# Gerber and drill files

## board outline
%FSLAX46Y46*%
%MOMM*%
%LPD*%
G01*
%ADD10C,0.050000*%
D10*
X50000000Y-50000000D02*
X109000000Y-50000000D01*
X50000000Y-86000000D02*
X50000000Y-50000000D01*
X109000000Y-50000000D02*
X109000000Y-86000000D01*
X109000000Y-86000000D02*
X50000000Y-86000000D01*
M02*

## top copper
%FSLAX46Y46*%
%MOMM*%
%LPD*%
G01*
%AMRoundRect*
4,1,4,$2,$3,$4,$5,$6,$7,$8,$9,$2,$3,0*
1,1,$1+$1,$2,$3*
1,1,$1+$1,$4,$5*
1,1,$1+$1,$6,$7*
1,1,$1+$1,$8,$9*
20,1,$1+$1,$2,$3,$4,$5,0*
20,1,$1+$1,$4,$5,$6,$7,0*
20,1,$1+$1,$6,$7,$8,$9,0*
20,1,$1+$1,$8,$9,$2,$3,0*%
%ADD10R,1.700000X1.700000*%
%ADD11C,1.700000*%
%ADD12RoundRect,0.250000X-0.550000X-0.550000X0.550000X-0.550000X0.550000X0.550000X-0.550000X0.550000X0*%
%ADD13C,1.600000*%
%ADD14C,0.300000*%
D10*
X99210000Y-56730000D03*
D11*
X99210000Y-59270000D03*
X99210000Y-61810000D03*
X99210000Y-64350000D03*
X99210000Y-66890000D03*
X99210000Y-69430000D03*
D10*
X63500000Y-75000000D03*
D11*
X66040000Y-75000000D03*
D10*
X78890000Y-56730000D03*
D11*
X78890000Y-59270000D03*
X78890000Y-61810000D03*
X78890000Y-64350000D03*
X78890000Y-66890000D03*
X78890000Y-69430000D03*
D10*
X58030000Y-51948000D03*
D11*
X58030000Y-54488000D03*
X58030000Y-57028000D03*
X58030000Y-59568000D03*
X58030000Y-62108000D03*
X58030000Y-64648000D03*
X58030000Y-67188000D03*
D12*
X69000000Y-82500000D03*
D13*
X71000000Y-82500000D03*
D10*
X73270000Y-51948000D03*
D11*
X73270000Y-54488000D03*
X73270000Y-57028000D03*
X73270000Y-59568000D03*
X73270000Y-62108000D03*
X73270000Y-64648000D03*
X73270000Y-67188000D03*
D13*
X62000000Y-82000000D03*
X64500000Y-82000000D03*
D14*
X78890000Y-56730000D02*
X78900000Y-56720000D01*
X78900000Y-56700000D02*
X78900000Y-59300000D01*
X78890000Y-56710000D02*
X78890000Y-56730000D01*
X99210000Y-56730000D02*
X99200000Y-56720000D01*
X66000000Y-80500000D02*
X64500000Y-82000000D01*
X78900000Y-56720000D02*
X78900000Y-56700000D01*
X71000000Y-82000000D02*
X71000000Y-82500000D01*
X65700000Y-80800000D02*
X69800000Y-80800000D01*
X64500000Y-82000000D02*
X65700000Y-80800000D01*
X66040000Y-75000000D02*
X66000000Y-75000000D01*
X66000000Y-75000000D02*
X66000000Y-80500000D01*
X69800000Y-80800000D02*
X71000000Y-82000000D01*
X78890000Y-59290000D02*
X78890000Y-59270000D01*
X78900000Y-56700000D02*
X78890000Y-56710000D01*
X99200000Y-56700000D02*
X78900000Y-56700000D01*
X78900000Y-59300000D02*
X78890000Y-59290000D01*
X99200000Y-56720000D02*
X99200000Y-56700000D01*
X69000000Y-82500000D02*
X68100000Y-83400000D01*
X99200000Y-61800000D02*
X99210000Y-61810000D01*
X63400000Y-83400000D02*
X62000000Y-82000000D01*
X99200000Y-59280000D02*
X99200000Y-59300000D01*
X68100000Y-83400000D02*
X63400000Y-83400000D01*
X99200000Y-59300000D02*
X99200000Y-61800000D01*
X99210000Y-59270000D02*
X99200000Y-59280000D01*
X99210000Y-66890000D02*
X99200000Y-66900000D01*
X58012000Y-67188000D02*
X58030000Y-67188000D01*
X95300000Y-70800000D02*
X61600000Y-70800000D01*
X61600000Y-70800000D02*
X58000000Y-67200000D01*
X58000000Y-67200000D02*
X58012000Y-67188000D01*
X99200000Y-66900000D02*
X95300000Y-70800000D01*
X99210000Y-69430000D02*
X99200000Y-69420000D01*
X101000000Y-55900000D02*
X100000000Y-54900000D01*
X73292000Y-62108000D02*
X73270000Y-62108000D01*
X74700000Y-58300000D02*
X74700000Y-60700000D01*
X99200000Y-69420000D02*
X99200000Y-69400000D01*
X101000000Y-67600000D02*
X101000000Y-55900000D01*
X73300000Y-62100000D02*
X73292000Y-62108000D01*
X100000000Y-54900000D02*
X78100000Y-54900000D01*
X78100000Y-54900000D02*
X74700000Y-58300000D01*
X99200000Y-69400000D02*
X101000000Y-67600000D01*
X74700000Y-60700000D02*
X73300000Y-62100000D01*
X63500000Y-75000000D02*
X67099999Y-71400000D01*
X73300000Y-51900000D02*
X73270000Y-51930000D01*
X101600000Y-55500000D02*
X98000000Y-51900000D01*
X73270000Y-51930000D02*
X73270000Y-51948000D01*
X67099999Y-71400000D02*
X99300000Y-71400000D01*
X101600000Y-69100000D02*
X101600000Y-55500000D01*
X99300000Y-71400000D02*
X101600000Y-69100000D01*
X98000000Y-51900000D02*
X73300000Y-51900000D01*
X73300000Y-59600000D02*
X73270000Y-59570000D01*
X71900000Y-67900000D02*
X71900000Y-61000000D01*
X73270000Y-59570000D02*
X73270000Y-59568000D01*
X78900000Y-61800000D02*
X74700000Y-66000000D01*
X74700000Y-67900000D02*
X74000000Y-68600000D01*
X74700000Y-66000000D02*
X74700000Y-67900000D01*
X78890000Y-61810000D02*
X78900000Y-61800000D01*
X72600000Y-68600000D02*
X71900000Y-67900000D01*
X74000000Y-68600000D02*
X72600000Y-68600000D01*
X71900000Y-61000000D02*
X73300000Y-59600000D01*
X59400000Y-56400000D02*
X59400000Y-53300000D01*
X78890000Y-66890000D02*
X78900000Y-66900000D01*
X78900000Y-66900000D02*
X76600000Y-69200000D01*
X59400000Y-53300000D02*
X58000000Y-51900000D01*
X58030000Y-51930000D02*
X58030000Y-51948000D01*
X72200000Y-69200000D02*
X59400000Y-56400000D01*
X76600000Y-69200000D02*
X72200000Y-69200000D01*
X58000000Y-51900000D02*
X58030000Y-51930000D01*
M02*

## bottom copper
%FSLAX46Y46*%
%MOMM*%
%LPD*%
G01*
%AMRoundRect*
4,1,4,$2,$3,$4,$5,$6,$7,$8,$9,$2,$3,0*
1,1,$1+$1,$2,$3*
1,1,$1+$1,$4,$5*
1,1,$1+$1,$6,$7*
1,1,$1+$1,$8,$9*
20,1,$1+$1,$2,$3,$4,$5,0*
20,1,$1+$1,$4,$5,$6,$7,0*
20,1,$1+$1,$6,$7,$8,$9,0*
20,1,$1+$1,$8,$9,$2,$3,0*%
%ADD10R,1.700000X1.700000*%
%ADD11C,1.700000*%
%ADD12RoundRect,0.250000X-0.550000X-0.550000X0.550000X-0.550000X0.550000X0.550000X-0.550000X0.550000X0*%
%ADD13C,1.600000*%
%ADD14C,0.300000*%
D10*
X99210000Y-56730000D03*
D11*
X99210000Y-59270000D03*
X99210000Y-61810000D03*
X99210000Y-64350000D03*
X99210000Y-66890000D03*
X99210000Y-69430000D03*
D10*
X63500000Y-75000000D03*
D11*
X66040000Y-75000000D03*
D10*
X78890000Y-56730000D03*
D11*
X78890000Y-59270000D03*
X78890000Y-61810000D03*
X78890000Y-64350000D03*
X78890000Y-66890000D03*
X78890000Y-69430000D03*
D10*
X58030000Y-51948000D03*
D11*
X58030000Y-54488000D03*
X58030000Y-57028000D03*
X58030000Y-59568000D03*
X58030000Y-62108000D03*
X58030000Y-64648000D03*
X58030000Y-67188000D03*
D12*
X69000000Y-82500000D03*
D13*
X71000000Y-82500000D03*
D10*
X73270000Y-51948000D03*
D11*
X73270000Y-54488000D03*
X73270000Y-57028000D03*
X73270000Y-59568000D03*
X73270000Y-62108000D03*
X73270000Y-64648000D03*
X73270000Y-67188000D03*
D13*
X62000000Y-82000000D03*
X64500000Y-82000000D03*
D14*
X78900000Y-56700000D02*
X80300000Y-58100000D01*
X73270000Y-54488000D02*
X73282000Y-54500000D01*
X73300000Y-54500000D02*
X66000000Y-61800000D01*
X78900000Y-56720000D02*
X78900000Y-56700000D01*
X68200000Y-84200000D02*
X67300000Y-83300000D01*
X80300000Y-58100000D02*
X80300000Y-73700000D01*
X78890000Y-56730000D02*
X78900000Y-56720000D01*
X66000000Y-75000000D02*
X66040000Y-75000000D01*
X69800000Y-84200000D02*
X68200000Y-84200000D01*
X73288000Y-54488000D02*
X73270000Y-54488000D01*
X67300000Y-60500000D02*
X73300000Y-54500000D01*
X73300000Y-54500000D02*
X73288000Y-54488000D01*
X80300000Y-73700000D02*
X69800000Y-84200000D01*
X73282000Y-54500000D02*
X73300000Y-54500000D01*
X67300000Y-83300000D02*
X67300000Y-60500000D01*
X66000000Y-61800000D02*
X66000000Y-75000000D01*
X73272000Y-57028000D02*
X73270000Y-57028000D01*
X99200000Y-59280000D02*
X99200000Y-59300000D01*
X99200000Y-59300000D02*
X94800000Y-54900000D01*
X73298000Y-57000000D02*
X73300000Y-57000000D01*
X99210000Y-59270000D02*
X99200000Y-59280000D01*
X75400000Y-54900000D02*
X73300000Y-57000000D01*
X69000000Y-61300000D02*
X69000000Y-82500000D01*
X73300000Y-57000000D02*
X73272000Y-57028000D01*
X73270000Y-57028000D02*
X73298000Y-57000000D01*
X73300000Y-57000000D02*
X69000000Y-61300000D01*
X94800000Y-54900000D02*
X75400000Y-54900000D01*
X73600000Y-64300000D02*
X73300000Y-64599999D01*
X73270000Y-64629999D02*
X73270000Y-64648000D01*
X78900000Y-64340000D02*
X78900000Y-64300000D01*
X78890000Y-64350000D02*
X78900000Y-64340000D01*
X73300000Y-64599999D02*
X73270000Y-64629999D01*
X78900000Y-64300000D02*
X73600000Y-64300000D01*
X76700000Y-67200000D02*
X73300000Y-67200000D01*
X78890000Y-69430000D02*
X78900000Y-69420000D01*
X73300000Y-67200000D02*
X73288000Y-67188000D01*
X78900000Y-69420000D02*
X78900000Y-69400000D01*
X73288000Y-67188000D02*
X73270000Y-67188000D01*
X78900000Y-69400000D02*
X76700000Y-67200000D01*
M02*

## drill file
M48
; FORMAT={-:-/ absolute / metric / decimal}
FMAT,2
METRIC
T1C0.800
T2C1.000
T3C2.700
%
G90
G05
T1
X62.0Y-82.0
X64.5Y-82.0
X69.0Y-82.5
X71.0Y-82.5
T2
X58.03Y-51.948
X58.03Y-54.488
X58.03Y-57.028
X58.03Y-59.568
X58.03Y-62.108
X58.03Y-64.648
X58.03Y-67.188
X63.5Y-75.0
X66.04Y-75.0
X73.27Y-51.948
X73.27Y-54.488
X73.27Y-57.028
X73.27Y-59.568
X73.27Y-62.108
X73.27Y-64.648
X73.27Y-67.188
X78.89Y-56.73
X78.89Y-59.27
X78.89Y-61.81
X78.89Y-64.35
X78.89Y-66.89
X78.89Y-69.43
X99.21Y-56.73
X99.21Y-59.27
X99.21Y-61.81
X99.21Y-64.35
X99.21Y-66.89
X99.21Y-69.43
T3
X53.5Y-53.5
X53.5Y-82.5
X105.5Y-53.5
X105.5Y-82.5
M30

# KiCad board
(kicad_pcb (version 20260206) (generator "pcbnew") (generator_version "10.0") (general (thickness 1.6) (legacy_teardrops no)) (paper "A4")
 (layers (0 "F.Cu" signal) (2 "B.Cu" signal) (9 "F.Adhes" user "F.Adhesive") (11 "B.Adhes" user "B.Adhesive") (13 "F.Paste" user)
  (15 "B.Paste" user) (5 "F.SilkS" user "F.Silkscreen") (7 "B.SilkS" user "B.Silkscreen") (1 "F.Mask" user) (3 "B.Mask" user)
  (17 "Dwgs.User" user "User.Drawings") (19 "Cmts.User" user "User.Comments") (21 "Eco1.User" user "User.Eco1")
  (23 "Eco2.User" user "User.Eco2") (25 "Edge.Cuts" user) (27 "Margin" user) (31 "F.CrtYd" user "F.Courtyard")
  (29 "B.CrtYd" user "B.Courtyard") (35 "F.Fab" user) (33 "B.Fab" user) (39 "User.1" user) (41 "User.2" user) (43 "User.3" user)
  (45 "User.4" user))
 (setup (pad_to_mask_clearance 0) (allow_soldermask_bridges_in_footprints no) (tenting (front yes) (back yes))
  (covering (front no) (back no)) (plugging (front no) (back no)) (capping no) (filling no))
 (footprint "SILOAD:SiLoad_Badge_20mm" (layer "F.Cu") (at 89.05 82)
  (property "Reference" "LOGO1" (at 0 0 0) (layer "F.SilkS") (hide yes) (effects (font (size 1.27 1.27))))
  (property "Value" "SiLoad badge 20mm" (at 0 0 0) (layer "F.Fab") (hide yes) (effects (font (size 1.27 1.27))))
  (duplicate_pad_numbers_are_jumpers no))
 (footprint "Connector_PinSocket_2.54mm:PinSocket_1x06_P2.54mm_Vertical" (layer "F.Cu") (at 99.21 56.73)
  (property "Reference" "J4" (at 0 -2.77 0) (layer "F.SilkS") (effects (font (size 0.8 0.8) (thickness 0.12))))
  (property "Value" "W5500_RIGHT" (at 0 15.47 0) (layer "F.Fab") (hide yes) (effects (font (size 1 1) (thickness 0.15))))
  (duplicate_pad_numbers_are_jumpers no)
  (pad "1" thru_hole rect (at 0 0) (size 1.7 1.7) (drill 1) (layers "*.Cu" "*.Mask") (remove_unused_layers no) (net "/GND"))
  (pad "2" thru_hole circle (at 0 2.54) (size 1.7 1.7) (drill 1) (layers "*.Cu" "*.Mask") (remove_unused_layers no) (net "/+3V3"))
  (pad "3" thru_hole circle (at 0 5.08) (size 1.7 1.7) (drill 1) (layers "*.Cu" "*.Mask") (remove_unused_layers no) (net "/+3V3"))
  (pad "4" thru_hole circle (at 0 7.62) (size 1.7 1.7) (drill 1) (layers "*.Cu" "*.Mask") (remove_unused_layers no))
  (pad "5" thru_hole circle (at 0 10.16) (size 1.7 1.7) (drill 1) (layers "*.Cu" "*.Mask") (remove_unused_layers no) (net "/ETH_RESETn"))
  (pad "6" thru_hole circle (at 0 12.7) (size 1.7 1.7) (drill 1) (layers "*.Cu" "*.Mask") (remove_unused_layers no) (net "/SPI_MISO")))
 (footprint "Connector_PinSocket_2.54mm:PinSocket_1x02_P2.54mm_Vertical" (layer "F.Cu") (at 63.5 75 90)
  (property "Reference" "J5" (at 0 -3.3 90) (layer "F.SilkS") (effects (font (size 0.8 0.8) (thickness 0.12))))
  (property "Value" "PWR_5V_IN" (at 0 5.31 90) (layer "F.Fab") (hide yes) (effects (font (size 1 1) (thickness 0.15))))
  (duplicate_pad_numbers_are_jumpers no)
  (pad "1" thru_hole rect (at 0 0 90) (size 1.7 1.7) (drill 1) (layers "*.Cu" "*.Mask") (remove_unused_layers no) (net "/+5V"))
  (pad "2" thru_hole circle (at 0 2.54 90) (size 1.7 1.7) (drill 1) (layers "*.Cu" "*.Mask") (remove_unused_layers no) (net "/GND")))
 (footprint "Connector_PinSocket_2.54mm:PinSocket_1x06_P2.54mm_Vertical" (layer "F.Cu") (at 78.89 56.73)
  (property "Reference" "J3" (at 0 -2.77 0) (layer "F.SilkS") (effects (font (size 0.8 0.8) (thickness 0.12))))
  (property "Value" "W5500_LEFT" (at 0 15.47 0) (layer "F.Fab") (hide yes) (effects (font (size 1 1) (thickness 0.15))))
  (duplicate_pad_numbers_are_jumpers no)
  (pad "1" thru_hole rect (at 0 0) (size 1.7 1.7) (drill 1) (layers "*.Cu" "*.Mask") (remove_unused_layers no) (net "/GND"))
  (pad "2" thru_hole circle (at 0 2.54) (size 1.7 1.7) (drill 1) (layers "*.Cu" "*.Mask") (remove_unused_layers no) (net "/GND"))
  (pad "3" thru_hole circle (at 0 5.08) (size 1.7 1.7) (drill 1) (layers "*.Cu" "*.Mask") (remove_unused_layers no) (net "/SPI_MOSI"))
  (pad "4" thru_hole circle (at 0 7.62) (size 1.7 1.7) (drill 1) (layers "*.Cu" "*.Mask") (remove_unused_layers no) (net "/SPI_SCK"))
  (pad "5" thru_hole circle (at 0 10.16) (size 1.7 1.7) (drill 1) (layers "*.Cu" "*.Mask") (remove_unused_layers no) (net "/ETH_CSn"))
  (pad "6" thru_hole circle (at 0 12.7) (size 1.7 1.7) (drill 1) (layers "*.Cu" "*.Mask") (remove_unused_layers no) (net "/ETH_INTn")))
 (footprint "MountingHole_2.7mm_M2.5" (layer "F.Cu") (at 105.5 53.5)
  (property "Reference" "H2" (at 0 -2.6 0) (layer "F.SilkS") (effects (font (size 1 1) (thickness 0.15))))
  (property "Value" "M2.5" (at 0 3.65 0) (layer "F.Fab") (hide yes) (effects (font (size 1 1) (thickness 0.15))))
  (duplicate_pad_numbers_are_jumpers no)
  (pad "" np_thru_hole circle (at 0 0) (size 2.7 2.7) (drill 2.7) (layers "*.Cu" "*.Mask")))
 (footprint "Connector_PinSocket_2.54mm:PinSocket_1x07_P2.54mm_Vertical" (layer "F.Cu") (at 58.03 51.948)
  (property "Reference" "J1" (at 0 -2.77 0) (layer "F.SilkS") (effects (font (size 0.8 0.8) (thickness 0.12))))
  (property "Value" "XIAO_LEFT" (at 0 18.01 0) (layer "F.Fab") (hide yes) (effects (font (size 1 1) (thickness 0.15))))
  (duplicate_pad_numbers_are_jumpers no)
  (pad "1" thru_hole rect (at 0 0) (size 1.7 1.7) (drill 1) (layers "*.Cu" "*.Mask") (remove_unused_layers no) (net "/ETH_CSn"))
  (pad "2" thru_hole circle (at 0 2.54) (size 1.7 1.7) (drill 1) (layers "*.Cu" "*.Mask") (remove_unused_layers no))
  (pad "3" thru_hole circle (at 0 5.08) (size 1.7 1.7) (drill 1) (layers "*.Cu" "*.Mask") (remove_unused_layers no))
  (pad "4" thru_hole circle (at 0 7.62) (size 1.7 1.7) (drill 1) (layers "*.Cu" "*.Mask") (remove_unused_layers no))
  (pad "5" thru_hole circle (at 0 10.16) (size 1.7 1.7) (drill 1) (layers "*.Cu" "*.Mask") (remove_unused_layers no))
  (pad "6" thru_hole circle (at 0 12.7) (size 1.7 1.7) (drill 1) (layers "*.Cu" "*.Mask") (remove_unused_layers no))
  (pad "7" thru_hole circle (at 0 15.24) (size 1.7 1.7) (drill 1) (layers "*.Cu" "*.Mask") (remove_unused_layers no) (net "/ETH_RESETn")))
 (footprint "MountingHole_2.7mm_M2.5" (layer "F.Cu") (at 105.5 82.5)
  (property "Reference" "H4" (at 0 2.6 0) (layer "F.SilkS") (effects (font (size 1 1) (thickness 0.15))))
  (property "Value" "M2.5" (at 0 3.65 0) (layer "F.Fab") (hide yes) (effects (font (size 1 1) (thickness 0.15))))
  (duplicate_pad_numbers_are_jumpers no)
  (pad "" np_thru_hole circle (at 0 0) (size 2.7 2.7) (drill 2.7) (layers "*.Cu" "*.Mask")))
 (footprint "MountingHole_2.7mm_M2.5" (layer "F.Cu") (at 53.5 53.5)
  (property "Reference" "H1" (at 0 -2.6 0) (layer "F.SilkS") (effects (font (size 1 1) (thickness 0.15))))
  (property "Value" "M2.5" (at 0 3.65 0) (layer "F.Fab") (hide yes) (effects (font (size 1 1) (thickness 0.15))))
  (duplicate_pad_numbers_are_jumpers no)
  (pad "" np_thru_hole circle (at 0 0) (size 2.7 2.7) (drill 2.7) (layers "*.Cu" "*.Mask")))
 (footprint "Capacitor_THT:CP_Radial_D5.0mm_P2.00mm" (layer "F.Cu") (at 69 82.5)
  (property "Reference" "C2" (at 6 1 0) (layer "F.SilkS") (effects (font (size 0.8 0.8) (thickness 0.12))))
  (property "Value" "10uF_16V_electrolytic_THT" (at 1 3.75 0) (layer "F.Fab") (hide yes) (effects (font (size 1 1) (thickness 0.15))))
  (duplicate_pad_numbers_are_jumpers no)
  (pad "1" thru_hole roundrect (at 0 0) (size 1.6 1.6) (drill 0.8) (layers "*.Cu" "*.Mask") (remove_unused_layers no)
   (roundrect_rratio 0.15625) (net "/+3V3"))
  (pad "2" thru_hole circle (at 2 0) (size 1.6 1.6) (drill 0.8) (layers "*.Cu" "*.Mask") (remove_unused_layers no) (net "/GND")))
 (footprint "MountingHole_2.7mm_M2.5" (layer "F.Cu") (at 53.5 82.5)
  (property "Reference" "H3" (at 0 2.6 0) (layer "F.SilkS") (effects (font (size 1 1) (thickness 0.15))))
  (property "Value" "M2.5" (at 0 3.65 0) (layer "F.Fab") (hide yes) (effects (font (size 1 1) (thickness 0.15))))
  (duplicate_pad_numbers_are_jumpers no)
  (pad "" np_thru_hole circle (at 0 0) (size 2.7 2.7) (drill 2.7) (layers "*.Cu" "*.Mask")))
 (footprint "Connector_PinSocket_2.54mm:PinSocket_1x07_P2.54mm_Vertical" (layer "F.Cu") (at 73.27 51.948)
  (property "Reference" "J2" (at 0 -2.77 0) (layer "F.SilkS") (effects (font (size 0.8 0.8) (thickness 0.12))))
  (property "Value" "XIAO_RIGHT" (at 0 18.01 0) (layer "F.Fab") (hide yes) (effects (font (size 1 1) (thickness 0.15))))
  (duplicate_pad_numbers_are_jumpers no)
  (pad "1" thru_hole rect (at 0 0) (size 1.7 1.7) (drill 1) (layers "*.Cu" "*.Mask") (remove_unused_layers no) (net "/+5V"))
  (pad "2" thru_hole circle (at 0 2.54) (size 1.7 1.7) (drill 1) (layers "*.Cu" "*.Mask") (remove_unused_layers no) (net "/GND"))
  (pad "3" thru_hole circle (at 0 5.08) (size 1.7 1.7) (drill 1) (layers "*.Cu" "*.Mask") (remove_unused_layers no) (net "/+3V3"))
  (pad "4" thru_hole circle (at 0 7.62) (size 1.7 1.7) (drill 1) (layers "*.Cu" "*.Mask") (remove_unused_layers no) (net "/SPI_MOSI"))
  (pad "5" thru_hole circle (at 0 10.16) (size 1.7 1.7) (drill 1) (layers "*.Cu" "*.Mask") (remove_unused_layers no) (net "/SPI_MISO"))
  (pad "6" thru_hole circle (at 0 12.7) (size 1.7 1.7) (drill 1) (layers "*.Cu" "*.Mask") (remove_unused_layers no) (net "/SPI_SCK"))
  (pad "7" thru_hole circle (at 0 15.24) (size 1.7 1.7) (drill 1) (layers "*.Cu" "*.Mask") (remove_unused_layers no) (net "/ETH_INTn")))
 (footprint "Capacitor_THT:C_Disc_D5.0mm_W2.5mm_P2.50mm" (layer "F.Cu") (at 62 82)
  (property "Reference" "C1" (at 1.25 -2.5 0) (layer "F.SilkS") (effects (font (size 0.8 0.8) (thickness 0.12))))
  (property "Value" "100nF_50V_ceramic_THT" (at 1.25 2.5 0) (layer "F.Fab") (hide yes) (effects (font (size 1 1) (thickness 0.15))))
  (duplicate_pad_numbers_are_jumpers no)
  (pad "1" thru_hole circle (at 0 0) (size 1.6 1.6) (drill 0.8) (layers "*.Cu" "*.Mask") (remove_unused_layers no) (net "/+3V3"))
  (pad "2" thru_hole circle (at 2.5 0) (size 1.6 1.6) (drill 0.8) (layers "*.Cu" "*.Mask") (remove_unused_layers no) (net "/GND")))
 (gr_line (start 50 50) (end 109 50) (stroke (width 0.05) (type default)) (layer "Edge.Cuts"))
 (gr_line (start 50 86) (end 50 50) (stroke (width 0.05) (type default)) (layer "Edge.Cuts"))
 (gr_line (start 109 50) (end 109 86) (stroke (width 0.05) (type default)) (layer "Edge.Cuts"))
 (gr_line (start 109 86) (end 50 86) (stroke (width 0.05) (type default)) (layer "Edge.Cuts"))
 (segment (start 78.89 56.73) (end 78.9 56.72) (width 0.3) (layer "F.Cu") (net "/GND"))
 (segment (start 78.9 56.7) (end 78.9 59.3) (width 0.3) (layer "F.Cu") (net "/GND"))
 (segment (start 78.89 56.71) (end 78.89 56.73) (width 0.3) (layer "F.Cu") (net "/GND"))
 (segment (start 99.21 56.73) (end 99.2 56.72) (width 0.3) (layer "F.Cu") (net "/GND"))
 (segment (start 66 80.5) (end 64.5 82) (width 0.3) (layer "F.Cu") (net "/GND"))
 (segment (start 78.9 56.72) (end 78.9 56.7) (width 0.3) (layer "F.Cu") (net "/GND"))
 (segment (start 71 82) (end 71 82.5) (width 0.3) (layer "F.Cu") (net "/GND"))
 (segment (start 65.7 80.8) (end 69.8 80.8) (width 0.3) (layer "F.Cu") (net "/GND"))
 (segment (start 64.5 82) (end 65.7 80.8) (width 0.3) (layer "F.Cu") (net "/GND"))
 (segment (start 66.04 75) (end 66 75) (width 0.3) (layer "F.Cu") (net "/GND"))
 (segment (start 66 75) (end 66 80.5) (width 0.3) (layer "F.Cu") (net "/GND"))
 (segment (start 69.8 80.8) (end 71 82) (width 0.3) (layer "F.Cu") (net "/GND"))
 (segment (start 78.89 59.29) (end 78.89 59.27) (width 0.3) (layer "F.Cu") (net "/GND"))
 (segment (start 78.9 56.7) (end 78.89 56.71) (width 0.3) (layer "F.Cu") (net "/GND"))
 (segment (start 99.2 56.7) (end 78.9 56.7) (width 0.3) (layer "F.Cu") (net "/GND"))
 (segment (start 78.9 59.3) (end 78.89 59.29) (width 0.3) (layer "F.Cu") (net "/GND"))
 (segment (start 99.2 56.72) (end 99.2 56.7) (width 0.3) (layer "F.Cu") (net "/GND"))
 (segment (start 78.9 56.7) (end 80.3 58.1) (width 0.3) (layer "B.Cu") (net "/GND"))
 (segment (start 73.27 54.488) (end 73.282 54.5) (width 0.3) (layer "B.Cu") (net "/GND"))
 (segment (start 73.3 54.5) (end 66 61.8) (width 0.3) (layer "B.Cu") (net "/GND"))
 (segment (start 78.9 56.72) (end 78.9 56.7) (width 0.3) (layer "B.Cu") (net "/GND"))
 (segment (start 68.2 84.2) (end 67.3 83.3) (width 0.3) (layer "B.Cu") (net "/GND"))
 (segment (start 80.3 58.1) (end 80.3 73.7) (width 0.3) (layer "B.Cu") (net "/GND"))
 (segment (start 78.89 56.73) (end 78.9 56.72) (width 0.3) (layer "B.Cu") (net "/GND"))
 (segment (start 66 75) (end 66.04 75) (width 0.3) (layer "B.Cu") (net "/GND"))
 (segment (start 69.8 84.2) (end 68.2 84.2) (width 0.3) (layer "B.Cu") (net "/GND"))
 (segment (start 73.288 54.488) (end 73.27 54.488) (width 0.3) (layer "B.Cu") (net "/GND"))
 (segment (start 67.3 60.5) (end 73.3 54.5) (width 0.3) (layer "B.Cu") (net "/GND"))
 (segment (start 73.3 54.5) (end 73.288 54.488) (width 0.3) (layer "B.Cu") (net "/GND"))
 (segment (start 80.3 73.7) (end 69.8 84.2) (width 0.3) (layer "B.Cu") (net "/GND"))
 (segment (start 73.282 54.5) (end 73.3 54.5) (width 0.3) (layer "B.Cu") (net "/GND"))
 (segment (start 67.3 83.3) (end 67.3 60.5) (width 0.3) (layer "B.Cu") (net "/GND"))
 (segment (start 66 61.8) (end 66 75) (width 0.3) (layer "B.Cu") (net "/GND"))
 (segment (start 69 82.5) (end 68.1 83.4) (width 0.3) (layer "F.Cu") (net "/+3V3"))
 (segment (start 99.2 61.8) (end 99.21 61.81) (width 0.3) (layer "F.Cu") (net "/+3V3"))
 (segment (start 63.4 83.4) (end 62 82) (width 0.3) (layer "F.Cu") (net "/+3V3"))
 (segment (start 99.2 59.28) (end 99.2 59.3) (width 0.3) (layer "F.Cu") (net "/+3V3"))
 (segment (start 68.1 83.4) (end 63.4 83.4) (width 0.3) (layer "F.Cu") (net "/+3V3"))
 (segment (start 99.2 59.3) (end 99.2 61.8) (width 0.3) (layer "F.Cu") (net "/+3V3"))
 (segment (start 99.21 59.27) (end 99.2 59.28) (width 0.3) (layer "F.Cu") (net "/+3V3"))
 (segment (start 73.272 57.028) (end 73.27 57.028) (width 0.3) (layer "B.Cu") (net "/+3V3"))
 (segment (start 99.2 59.28) (end 99.2 59.3) (width 0.3) (layer "B.Cu") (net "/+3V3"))
 (segment (start 99.2 59.3) (end 94.8 54.9) (width 0.3) (layer "B.Cu") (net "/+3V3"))
 (segment (start 73.298 57) (end 73.3 57) (width 0.3) (layer "B.Cu") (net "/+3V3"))
 (segment (start 99.21 59.27) (end 99.2 59.28) (width 0.3) (layer "B.Cu") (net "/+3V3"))
 (segment (start 75.4 54.9) (end 73.3 57) (width 0.3) (layer "B.Cu") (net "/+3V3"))
 (segment (start 69 61.3) (end 69 82.5) (width 0.3) (layer "B.Cu") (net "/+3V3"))
 (segment (start 73.3 57) (end 73.272 57.028) (width 0.3) (layer "B.Cu") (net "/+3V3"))
 (segment (start 73.27 57.028) (end 73.298 57) (width 0.3) (layer "B.Cu") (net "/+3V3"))
 (segment (start 73.3 57) (end 69 61.3) (width 0.3) (layer "B.Cu") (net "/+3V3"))
 (segment (start 94.8 54.9) (end 75.4 54.9) (width 0.3) (layer "B.Cu") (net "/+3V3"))
 (segment (start 99.21 66.89) (end 99.2 66.9) (width 0.3) (layer "F.Cu") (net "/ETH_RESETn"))
 (segment (start 58.012 67.188) (end 58.03 67.188) (width 0.3) (layer "F.Cu") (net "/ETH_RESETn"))
 (segment (start 95.3 70.8) (end 61.6 70.8) (width 0.3) (layer "F.Cu") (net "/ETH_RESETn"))
 (segment (start 61.6 70.8) (end 58 67.2) (width 0.3) (layer "F.Cu") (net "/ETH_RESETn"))
 (segment (start 58 67.2) (end 58.012 67.188) (width 0.3) (layer "F.Cu") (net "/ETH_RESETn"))
 (segment (start 99.2 66.9) (end 95.3 70.8) (width 0.3) (layer "F.Cu") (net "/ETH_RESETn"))
 (segment (start 99.21 69.43) (end 99.2 69.42) (width 0.3) (layer "F.Cu") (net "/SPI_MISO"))
 (segment (start 101 55.9) (end 100 54.9) (width 0.3) (layer "F.Cu") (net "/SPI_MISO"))
 (segment (start 73.292 62.108) (end 73.27 62.108) (width 0.3) (layer "F.Cu") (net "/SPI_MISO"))
 (segment (start 74.7 58.3) (end 74.7 60.7) (width 0.3) (layer "F.Cu") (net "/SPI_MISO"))
 (segment (start 99.2 69.42) (end 99.2 69.4) (width 0.3) (layer "F.Cu") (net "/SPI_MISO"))
 (segment (start 101 67.6) (end 101 55.9) (width 0.3) (layer "F.Cu") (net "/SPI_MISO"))
 (segment (start 73.3 62.1) (end 73.292 62.108) (width 0.3) (layer "F.Cu") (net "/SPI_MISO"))
 (segment (start 100 54.9) (end 78.1 54.9) (width 0.3) (layer "F.Cu") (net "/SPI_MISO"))
 (segment (start 78.1 54.9) (end 74.7 58.3) (width 0.3) (layer "F.Cu") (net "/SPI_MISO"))
 (segment (start 99.2 69.4) (end 101 67.6) (width 0.3) (layer "F.Cu") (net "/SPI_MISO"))
 (segment (start 74.7 60.7) (end 73.3 62.1) (width 0.3) (layer "F.Cu") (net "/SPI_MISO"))
 (segment (start 63.5 75) (end 67.099999 71.4) (width 0.3) (layer "F.Cu") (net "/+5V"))
 (segment (start 73.3 51.9) (end 73.27 51.93) (width 0.3) (layer "F.Cu") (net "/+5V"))
 (segment (start 101.6 55.5) (end 98 51.9) (width 0.3) (layer "F.Cu") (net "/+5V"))
 (segment (start 73.27 51.93) (end 73.27 51.948) (width 0.3) (layer "F.Cu") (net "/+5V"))
 (segment (start 67.099999 71.4) (end 99.3 71.4) (width 0.3) (layer "F.Cu") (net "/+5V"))
 (segment (start 101.6 69.1) (end 101.6 55.5) (width 0.3) (layer "F.Cu") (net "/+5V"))
 (segment (start 99.3 71.4) (end 101.6 69.1) (width 0.3) (layer "F.Cu") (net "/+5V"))
 (segment (start 98 51.9) (end 73.3 51.9) (width 0.3) (layer "F.Cu") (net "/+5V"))
 (segment (start 73.3 59.6) (end 73.27 59.57) (width 0.3) (layer "F.Cu") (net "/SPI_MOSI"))
 (segment (start 71.9 67.9) (end 71.9 61) (width 0.3) (layer "F.Cu") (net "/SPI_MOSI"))
 (segment (start 73.27 59.57) (end 73.27 59.568) (width 0.3) (layer "F.Cu") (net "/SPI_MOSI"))
 (segment (start 78.9 61.8) (end 74.7 66) (width 0.3) (layer "F.Cu") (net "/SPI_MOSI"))
 (segment (start 74.7 67.9) (end 74 68.6) (width 0.3) (layer "F.Cu") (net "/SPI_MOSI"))
 (segment (start 74.7 66) (end 74.7 67.9) (width 0.3) (layer "F.Cu") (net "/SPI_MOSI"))
 (segment (start 78.89 61.81) (end 78.9 61.8) (width 0.3) (layer "F.Cu") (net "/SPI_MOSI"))
 (segment (start 72.6 68.6) (end 71.9 67.9) (width 0.3) (layer "F.Cu") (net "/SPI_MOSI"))
 (segment (start 74 68.6) (end 72.6 68.6) (width 0.3) (layer "F.Cu") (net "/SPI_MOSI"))
 (segment (start 71.9 61) (end 73.3 59.6) (width 0.3) (layer "F.Cu") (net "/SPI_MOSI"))
 (segment (start 73.6 64.3) (end 73.3 64.599999) (width 0.3) (layer "B.Cu") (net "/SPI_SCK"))
 (segment (start 73.27 64.629999) (end 73.27 64.648) (width 0.3) (layer "B.Cu") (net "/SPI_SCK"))
 (segment (start 78.9 64.34) (end 78.9 64.3) (width 0.3) (layer "B.Cu") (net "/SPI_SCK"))
 (segment (start 78.89 64.35) (end 78.9 64.34) (width 0.3) (layer "B.Cu") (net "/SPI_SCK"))
 (segment (start 73.3 64.599999) (end 73.27 64.629999) (width 0.3) (layer "B.Cu") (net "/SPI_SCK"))
 (segment (start 78.9 64.3) (end 73.6 64.3) (width 0.3) (layer "B.Cu") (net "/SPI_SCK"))
 (segment (start 59.4 56.4) (end 59.4 53.3) (width 0.3) (layer "F.Cu") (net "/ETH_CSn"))
 (segment (start 78.89 66.89) (end 78.9 66.9) (width 0.3) (layer "F.Cu") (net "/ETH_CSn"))
 (segment (start 78.9 66.9) (end 76.6 69.2) (width 0.3) (layer "F.Cu") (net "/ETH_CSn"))
 (segment (start 59.4 53.3) (end 58 51.9) (width 0.3) (layer "F.Cu") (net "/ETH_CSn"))
 (segment (start 58.03 51.93) (end 58.03 51.948) (width 0.3) (layer "F.Cu") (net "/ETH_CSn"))
 (segment (start 72.2 69.2) (end 59.4 56.4) (width 0.3) (layer "F.Cu") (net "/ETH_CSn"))
 (segment (start 76.6 69.2) (end 72.2 69.2) (width 0.3) (layer "F.Cu") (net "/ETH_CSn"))
 (segment (start 58 51.9) (end 58.03 51.93) (width 0.3) (layer "F.Cu") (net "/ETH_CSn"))
 (segment (start 76.7 67.2) (end 73.3 67.2) (width 0.3) (layer "B.Cu") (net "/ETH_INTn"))
 (segment (start 78.89 69.43) (end 78.9 69.42) (width 0.3) (layer "B.Cu") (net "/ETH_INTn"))
 (segment (start 73.3 67.2) (end 73.288 67.188) (width 0.3) (layer "B.Cu") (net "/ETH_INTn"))
 (segment (start 78.9 69.42) (end 78.9 69.4) (width 0.3) (layer "B.Cu") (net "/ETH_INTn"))
 (segment (start 73.288 67.188) (end 73.27 67.188) (width 0.3) (layer "B.Cu") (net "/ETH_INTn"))
 (segment (start 78.9 69.4) (end 76.7 67.2) (width 0.3) (layer "B.Cu") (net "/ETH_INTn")))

